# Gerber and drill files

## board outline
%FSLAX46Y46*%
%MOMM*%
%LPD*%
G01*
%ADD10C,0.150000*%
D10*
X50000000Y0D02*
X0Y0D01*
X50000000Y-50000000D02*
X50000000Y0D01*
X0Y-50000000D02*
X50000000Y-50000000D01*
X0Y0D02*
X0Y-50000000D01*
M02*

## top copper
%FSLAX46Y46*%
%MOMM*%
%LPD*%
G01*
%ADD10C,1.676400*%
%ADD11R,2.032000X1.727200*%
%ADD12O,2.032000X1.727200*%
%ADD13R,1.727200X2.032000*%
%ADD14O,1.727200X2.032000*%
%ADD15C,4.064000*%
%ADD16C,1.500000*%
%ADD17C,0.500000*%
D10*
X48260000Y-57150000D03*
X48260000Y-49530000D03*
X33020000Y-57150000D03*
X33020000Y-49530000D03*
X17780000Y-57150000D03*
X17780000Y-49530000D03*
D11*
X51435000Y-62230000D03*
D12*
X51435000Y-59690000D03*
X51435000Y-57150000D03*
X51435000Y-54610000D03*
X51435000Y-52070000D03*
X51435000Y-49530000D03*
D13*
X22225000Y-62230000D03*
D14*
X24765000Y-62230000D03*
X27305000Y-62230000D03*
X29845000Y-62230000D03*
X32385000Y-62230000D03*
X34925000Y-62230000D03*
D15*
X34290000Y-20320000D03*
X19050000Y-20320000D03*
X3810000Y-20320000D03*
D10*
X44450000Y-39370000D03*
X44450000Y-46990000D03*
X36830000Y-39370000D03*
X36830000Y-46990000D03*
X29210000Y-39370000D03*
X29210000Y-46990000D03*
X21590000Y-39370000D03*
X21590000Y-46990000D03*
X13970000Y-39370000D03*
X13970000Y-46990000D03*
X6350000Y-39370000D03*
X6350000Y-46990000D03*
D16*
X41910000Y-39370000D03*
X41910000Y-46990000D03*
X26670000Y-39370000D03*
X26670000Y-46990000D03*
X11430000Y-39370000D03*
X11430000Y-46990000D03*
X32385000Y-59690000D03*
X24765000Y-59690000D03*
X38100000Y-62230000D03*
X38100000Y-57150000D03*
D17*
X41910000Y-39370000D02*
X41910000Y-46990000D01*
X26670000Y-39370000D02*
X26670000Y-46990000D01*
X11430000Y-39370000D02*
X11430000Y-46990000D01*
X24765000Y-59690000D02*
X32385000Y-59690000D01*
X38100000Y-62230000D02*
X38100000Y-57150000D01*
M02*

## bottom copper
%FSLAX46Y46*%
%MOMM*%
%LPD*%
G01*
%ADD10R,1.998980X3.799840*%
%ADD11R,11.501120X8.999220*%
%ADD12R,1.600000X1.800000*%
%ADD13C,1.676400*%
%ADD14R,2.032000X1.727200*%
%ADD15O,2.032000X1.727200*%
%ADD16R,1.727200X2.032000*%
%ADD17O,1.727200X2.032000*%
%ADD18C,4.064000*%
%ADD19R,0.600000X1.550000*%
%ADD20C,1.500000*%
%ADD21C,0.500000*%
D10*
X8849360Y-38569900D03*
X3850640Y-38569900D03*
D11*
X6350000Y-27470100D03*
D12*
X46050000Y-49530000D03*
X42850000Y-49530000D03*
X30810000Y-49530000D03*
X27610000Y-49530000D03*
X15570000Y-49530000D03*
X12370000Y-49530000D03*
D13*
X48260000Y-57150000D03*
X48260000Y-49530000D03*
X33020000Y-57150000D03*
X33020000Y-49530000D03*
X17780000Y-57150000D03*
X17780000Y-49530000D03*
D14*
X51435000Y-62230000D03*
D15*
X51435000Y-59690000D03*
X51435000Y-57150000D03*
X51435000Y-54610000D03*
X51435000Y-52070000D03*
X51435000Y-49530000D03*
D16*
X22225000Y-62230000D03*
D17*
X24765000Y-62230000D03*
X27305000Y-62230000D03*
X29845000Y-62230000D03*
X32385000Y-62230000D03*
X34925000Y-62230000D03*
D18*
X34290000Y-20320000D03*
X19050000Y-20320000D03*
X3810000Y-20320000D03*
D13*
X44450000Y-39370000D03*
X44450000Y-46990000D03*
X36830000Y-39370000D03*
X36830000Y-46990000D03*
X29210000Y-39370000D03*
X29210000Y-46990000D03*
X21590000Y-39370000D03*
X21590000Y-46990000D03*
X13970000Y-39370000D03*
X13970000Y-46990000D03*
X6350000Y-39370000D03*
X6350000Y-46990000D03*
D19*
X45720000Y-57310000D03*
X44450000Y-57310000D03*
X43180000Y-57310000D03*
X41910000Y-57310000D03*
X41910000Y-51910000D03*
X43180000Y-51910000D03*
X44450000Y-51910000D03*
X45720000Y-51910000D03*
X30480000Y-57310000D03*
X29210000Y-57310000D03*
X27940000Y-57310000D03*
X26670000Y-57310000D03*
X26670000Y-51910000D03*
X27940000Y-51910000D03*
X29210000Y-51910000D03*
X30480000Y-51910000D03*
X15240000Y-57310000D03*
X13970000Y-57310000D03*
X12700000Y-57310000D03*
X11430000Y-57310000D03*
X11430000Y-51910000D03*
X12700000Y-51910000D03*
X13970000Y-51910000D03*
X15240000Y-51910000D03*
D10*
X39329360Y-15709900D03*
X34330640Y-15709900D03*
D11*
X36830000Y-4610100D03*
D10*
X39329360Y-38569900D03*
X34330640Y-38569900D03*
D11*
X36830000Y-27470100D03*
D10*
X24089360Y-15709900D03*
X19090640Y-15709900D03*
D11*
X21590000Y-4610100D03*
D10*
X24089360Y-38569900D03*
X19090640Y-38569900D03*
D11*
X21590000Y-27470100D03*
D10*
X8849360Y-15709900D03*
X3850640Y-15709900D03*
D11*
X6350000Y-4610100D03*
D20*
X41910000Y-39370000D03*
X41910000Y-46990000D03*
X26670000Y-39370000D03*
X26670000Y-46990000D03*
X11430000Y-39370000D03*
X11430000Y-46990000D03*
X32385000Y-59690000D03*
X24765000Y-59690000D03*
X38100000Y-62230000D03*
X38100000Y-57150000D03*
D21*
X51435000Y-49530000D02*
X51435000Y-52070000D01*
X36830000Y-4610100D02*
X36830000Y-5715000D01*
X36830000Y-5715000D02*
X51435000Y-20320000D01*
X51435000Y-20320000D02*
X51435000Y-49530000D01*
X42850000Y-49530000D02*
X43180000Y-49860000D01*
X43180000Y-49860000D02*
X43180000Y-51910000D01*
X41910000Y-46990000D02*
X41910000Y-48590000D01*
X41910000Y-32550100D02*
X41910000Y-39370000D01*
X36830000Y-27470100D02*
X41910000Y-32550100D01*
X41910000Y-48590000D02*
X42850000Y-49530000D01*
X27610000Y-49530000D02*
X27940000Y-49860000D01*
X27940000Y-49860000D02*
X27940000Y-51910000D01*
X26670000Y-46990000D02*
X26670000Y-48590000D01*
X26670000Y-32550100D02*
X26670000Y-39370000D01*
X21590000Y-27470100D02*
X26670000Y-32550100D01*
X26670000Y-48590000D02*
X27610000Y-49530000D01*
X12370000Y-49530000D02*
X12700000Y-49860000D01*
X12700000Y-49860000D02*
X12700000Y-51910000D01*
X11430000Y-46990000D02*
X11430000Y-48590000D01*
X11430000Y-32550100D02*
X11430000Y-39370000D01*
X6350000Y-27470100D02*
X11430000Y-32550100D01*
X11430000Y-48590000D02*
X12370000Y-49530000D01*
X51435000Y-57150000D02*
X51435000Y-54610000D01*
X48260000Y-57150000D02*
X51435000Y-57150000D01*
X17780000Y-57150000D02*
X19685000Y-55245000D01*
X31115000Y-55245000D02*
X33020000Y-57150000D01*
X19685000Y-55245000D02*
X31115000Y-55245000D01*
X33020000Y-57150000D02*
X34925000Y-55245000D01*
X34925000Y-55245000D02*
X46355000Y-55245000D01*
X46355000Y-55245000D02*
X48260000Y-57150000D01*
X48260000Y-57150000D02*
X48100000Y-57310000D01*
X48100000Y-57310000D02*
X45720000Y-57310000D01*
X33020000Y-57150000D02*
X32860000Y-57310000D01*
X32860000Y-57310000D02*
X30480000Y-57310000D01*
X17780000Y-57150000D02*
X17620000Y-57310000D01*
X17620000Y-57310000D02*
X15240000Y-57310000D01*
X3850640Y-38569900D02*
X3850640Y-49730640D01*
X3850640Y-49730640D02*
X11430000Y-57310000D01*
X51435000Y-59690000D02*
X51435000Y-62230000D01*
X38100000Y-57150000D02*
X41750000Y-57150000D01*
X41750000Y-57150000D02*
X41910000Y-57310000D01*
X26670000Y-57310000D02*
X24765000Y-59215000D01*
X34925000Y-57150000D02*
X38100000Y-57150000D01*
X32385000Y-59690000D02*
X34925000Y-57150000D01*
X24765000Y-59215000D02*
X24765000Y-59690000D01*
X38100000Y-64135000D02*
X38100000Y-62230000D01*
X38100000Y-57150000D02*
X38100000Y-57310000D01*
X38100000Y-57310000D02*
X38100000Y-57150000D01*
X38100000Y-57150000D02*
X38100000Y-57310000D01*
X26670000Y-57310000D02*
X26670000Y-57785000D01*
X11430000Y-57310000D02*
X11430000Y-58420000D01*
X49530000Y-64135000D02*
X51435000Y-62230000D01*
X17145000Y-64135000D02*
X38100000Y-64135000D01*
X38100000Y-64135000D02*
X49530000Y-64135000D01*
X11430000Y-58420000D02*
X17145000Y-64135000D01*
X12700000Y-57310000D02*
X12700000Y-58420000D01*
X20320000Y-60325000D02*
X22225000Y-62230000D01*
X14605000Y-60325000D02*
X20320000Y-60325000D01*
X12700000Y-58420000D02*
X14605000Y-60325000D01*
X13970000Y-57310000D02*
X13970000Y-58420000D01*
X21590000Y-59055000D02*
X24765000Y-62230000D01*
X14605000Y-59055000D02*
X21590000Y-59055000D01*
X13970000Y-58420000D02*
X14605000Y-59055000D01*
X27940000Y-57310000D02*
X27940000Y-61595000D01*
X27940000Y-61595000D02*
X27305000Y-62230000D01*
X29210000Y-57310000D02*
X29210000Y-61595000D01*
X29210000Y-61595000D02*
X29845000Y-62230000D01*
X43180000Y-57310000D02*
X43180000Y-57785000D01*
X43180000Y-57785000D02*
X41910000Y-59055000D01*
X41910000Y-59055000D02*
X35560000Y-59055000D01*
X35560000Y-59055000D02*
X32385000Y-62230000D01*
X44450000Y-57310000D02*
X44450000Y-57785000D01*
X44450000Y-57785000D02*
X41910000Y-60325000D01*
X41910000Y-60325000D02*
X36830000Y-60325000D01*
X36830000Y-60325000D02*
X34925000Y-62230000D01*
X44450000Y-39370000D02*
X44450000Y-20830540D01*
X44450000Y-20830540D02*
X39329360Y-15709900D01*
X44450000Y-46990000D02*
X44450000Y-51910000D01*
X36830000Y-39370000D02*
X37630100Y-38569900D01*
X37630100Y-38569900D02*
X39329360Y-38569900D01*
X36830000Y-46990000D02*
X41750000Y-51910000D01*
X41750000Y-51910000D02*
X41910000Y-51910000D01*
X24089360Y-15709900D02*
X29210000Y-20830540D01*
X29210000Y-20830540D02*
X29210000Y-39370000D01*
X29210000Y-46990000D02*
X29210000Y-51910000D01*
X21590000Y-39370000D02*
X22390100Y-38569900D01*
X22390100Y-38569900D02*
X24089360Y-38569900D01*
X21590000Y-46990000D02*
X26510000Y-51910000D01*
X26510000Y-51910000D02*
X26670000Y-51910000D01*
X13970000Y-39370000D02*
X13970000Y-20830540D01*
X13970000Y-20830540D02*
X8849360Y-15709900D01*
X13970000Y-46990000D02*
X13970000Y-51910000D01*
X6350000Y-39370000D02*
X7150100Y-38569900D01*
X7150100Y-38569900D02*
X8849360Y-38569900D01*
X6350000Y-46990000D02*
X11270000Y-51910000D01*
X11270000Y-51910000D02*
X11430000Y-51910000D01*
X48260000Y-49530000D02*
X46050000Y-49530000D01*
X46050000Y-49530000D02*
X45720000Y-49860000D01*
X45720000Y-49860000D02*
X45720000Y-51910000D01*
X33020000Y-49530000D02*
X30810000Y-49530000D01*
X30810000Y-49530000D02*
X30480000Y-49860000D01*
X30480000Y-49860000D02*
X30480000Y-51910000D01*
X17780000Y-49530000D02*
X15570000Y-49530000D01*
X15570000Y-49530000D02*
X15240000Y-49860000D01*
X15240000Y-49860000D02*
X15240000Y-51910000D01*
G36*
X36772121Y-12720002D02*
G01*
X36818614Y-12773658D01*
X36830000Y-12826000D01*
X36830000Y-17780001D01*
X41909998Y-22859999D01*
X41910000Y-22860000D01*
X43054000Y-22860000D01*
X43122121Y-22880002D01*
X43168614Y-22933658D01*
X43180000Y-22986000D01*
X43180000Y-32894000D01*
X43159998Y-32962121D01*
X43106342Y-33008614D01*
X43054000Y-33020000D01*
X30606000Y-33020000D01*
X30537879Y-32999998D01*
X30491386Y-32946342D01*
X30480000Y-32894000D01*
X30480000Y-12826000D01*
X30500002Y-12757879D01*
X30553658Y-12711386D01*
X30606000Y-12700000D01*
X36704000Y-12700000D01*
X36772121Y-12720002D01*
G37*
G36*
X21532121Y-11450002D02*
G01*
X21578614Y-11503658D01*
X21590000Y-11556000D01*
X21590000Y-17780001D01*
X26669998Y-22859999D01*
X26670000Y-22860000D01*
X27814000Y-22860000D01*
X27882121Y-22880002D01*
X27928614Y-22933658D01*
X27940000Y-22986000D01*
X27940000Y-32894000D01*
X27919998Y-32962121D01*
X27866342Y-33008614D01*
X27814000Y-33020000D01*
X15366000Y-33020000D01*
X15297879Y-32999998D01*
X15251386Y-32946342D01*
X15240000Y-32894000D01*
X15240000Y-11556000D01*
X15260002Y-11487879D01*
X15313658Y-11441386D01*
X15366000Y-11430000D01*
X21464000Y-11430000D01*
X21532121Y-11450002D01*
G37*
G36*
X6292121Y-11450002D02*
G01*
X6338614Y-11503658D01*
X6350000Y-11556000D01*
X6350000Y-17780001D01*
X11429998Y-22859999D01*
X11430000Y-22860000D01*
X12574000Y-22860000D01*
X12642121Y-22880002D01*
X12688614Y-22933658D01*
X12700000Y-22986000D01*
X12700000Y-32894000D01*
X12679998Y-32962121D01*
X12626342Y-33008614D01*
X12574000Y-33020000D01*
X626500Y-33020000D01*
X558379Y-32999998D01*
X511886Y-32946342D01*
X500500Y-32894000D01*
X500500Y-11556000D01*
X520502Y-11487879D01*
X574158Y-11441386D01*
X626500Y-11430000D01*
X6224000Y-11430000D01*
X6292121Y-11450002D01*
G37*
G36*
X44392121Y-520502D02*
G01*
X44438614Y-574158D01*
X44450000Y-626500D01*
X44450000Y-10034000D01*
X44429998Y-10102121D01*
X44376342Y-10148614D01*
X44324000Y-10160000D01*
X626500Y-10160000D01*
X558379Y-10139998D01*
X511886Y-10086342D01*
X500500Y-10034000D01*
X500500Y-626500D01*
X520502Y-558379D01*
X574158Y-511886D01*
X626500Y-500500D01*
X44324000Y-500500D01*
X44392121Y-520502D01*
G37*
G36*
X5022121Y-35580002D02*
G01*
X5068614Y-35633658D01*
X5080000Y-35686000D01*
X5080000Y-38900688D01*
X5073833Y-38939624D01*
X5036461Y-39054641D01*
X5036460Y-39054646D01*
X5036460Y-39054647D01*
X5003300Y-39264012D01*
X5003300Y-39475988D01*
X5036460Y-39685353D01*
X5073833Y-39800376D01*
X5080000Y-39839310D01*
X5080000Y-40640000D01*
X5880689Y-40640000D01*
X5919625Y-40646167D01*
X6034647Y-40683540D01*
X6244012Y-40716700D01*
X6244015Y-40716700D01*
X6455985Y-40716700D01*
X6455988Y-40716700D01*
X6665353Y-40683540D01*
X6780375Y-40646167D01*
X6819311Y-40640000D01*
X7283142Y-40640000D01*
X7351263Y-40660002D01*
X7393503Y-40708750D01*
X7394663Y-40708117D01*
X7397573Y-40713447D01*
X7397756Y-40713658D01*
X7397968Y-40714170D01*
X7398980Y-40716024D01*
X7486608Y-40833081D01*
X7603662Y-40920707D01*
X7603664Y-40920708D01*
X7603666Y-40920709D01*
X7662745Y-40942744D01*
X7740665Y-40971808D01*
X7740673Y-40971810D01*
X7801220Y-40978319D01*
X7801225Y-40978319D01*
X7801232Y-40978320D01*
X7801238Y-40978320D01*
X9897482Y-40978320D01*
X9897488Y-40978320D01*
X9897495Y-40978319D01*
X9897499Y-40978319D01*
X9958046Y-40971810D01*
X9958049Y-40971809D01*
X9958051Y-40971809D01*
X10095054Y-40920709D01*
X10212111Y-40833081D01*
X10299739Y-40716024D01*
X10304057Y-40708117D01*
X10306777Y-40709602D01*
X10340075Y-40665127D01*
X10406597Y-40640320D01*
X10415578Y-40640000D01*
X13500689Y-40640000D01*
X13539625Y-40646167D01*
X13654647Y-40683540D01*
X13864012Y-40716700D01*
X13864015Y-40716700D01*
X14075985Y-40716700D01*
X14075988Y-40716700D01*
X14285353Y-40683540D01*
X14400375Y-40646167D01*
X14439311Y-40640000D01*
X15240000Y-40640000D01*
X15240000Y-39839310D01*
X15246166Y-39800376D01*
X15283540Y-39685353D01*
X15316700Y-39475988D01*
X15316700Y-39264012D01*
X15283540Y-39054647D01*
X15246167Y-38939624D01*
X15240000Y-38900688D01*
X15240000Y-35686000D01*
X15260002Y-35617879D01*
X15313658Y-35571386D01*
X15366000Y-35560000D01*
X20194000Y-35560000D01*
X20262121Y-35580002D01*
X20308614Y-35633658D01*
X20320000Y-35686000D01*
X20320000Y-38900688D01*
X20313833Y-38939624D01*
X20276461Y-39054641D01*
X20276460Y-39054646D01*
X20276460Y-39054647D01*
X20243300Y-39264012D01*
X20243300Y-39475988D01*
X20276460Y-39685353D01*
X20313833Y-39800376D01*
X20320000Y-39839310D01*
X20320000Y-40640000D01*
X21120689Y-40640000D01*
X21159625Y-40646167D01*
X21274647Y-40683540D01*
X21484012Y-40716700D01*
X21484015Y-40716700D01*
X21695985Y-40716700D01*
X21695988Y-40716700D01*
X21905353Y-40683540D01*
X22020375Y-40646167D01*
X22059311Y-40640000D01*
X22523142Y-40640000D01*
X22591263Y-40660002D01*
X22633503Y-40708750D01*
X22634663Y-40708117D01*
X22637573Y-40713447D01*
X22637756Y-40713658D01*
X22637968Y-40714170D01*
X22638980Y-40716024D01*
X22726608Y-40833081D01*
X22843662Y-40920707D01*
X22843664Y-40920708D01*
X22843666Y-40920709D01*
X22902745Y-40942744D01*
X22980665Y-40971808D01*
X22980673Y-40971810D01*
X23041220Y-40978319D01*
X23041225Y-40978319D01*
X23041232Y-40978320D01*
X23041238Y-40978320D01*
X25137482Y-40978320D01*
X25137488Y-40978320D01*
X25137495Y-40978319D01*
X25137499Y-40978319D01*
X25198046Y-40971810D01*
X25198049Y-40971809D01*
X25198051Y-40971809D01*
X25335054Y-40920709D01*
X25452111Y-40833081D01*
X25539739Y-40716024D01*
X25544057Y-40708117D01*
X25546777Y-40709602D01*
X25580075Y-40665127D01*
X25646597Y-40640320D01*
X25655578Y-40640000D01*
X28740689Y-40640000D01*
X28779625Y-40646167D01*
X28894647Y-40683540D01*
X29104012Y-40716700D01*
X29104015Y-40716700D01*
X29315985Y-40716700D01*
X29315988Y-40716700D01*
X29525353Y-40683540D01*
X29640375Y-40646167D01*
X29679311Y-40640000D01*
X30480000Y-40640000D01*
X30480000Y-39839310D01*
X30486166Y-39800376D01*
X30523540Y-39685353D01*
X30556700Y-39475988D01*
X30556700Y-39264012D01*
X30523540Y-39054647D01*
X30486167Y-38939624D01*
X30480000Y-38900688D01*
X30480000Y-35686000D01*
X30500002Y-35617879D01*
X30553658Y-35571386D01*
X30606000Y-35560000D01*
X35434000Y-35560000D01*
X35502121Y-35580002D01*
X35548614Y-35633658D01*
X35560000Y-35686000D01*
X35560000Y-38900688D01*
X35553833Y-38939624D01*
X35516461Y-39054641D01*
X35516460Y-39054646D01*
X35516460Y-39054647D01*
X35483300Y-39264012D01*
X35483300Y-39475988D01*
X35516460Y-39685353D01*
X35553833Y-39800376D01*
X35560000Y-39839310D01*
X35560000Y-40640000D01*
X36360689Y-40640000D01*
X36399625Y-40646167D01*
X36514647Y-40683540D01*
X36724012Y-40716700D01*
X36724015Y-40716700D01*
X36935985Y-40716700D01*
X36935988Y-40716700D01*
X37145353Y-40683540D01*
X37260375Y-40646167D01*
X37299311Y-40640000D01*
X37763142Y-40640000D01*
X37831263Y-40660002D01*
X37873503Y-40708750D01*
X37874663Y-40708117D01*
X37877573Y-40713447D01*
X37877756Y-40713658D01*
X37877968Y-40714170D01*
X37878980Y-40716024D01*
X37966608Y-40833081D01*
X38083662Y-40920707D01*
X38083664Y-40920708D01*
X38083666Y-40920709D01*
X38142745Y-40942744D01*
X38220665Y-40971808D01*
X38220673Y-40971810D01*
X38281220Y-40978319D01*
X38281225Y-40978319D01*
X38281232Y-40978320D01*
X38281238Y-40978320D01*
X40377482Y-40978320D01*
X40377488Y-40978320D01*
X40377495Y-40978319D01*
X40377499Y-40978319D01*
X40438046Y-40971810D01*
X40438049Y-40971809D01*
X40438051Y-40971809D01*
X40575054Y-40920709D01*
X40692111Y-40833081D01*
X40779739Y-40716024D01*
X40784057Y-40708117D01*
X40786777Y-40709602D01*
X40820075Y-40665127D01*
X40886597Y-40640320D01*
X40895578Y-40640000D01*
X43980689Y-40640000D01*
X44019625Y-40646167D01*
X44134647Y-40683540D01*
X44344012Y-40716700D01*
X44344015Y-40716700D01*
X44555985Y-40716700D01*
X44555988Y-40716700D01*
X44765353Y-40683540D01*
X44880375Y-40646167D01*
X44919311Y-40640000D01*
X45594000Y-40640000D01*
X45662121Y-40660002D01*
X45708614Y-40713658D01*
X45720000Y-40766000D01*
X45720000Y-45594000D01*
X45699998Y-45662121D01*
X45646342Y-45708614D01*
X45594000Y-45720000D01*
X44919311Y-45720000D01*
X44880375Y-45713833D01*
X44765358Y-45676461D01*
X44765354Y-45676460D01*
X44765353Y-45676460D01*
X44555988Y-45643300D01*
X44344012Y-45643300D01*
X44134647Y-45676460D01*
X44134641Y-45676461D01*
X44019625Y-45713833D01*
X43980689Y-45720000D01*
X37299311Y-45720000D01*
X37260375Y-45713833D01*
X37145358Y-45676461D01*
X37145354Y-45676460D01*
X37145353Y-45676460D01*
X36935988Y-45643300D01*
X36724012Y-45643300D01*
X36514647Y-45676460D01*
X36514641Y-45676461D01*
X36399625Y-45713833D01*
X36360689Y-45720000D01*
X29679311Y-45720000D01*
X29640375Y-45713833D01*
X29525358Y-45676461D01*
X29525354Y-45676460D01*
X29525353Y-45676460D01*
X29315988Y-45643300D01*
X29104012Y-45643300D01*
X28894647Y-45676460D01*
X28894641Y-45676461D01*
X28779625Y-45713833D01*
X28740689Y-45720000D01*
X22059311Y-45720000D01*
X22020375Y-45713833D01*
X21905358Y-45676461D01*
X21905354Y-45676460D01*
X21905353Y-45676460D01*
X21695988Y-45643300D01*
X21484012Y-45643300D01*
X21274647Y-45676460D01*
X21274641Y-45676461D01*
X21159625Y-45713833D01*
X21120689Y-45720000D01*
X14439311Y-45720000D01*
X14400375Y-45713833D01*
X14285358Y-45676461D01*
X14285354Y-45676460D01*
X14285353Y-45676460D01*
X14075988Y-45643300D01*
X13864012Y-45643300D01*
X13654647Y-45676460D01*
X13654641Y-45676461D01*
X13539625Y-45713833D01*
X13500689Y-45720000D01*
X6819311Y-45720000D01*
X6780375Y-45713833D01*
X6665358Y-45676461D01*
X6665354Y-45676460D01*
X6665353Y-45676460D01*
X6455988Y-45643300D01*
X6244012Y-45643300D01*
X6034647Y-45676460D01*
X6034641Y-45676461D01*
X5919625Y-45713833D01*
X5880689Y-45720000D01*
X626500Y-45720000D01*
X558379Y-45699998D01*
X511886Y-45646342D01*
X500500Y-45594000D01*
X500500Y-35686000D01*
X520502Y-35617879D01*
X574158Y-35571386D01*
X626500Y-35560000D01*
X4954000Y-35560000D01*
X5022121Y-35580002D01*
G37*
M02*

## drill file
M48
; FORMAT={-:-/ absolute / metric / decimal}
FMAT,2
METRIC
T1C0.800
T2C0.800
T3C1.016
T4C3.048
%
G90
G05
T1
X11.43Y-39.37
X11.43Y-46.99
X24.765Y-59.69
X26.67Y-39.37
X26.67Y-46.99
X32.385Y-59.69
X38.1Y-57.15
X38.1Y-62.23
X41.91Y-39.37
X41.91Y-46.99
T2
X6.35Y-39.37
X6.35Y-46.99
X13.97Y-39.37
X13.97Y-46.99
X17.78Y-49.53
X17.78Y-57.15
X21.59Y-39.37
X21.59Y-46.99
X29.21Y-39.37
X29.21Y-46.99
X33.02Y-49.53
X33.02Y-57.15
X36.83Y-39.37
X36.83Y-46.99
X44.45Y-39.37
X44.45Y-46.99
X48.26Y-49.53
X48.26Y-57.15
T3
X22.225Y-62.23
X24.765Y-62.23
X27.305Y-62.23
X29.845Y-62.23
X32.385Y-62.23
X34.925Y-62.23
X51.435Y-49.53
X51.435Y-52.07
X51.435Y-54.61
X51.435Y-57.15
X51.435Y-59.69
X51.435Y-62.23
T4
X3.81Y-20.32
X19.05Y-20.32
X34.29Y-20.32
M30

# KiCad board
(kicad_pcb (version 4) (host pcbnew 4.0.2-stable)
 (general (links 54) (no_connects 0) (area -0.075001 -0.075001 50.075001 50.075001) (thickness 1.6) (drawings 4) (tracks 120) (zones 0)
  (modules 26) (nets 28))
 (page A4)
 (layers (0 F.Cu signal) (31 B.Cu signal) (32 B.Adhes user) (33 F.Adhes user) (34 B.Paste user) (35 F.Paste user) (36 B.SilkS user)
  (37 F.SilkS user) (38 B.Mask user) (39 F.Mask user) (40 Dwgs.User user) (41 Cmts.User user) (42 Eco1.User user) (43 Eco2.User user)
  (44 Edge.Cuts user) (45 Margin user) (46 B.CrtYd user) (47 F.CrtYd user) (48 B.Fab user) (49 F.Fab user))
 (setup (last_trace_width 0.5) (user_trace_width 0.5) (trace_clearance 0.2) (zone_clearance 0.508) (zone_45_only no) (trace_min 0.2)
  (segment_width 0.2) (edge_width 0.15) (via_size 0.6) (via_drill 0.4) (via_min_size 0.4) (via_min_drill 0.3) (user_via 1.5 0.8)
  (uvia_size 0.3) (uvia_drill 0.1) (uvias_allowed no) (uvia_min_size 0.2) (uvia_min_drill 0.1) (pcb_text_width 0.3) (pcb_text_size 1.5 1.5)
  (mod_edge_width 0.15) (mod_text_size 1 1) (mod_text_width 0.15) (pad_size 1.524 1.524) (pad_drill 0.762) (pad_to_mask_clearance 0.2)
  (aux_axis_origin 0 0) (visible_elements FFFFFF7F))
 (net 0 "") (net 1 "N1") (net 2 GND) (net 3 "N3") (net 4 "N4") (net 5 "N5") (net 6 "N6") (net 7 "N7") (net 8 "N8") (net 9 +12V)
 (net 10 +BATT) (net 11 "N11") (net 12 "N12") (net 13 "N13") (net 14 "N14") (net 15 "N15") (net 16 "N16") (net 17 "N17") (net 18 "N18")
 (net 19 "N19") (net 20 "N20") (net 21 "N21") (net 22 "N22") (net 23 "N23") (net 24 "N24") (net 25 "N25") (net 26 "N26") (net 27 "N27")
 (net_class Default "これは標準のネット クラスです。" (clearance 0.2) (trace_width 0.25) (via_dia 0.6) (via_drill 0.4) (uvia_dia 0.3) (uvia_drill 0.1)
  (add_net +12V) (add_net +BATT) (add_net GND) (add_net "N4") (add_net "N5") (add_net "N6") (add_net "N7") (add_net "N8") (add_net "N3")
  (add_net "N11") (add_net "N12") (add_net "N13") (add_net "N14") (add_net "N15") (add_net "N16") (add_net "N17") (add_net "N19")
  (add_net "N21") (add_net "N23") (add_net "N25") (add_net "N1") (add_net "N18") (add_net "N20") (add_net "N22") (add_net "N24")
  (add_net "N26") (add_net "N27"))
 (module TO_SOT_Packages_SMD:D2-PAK (layer B.Cu) (at 6.35 33.02 180)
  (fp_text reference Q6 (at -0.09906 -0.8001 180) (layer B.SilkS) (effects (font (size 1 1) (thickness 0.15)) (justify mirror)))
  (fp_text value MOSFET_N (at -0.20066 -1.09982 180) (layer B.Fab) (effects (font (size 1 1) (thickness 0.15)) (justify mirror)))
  (pad G smd rect (at -2.49936 -5.5499 180) (size 1.99898 3.79984) (layers B.Cu B.Paste B.Mask) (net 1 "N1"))
  (pad S smd rect (at 2.49936 -5.5499 180) (size 1.99898 3.79984) (layers B.Cu B.Paste B.Mask) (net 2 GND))
  (pad D smd rect (at 0 5.5499 180) (size 11.50112 8.99922) (layers B.Cu B.Paste B.Mask) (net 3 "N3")))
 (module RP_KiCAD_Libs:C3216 (layer B.Cu) (at 44.45 49.53 180)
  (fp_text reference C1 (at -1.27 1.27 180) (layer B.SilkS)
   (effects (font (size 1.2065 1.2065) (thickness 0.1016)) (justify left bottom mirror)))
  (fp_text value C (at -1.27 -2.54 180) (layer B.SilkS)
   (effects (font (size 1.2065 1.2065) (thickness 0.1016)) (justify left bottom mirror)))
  (pad 1 smd rect (at -1.6 0 180) (size 1.6 1.8) (layers B.Cu B.Paste B.Mask) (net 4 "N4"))
  (pad 2 smd rect (at 1.6 0 180) (size 1.6 1.8) (layers B.Cu B.Paste B.Mask) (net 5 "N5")))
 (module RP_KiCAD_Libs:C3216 (layer B.Cu) (at 29.21 49.53 180)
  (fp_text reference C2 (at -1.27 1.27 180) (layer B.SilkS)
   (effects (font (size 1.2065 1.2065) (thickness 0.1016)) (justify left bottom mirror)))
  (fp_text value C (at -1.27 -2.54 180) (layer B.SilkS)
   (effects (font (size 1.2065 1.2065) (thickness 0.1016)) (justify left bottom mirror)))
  (pad 1 smd rect (at -1.6 0 180) (size 1.6 1.8) (layers B.Cu B.Paste B.Mask) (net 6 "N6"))
  (pad 2 smd rect (at 1.6 0 180) (size 1.6 1.8) (layers B.Cu B.Paste B.Mask) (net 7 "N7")))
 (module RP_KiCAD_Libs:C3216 (layer B.Cu) (at 13.97 49.53 180)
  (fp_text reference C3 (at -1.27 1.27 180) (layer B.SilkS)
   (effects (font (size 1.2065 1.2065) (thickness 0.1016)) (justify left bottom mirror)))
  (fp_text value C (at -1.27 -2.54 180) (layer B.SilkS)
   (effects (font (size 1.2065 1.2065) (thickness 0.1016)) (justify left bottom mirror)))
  (pad 1 smd rect (at -1.6 0 180) (size 1.6 1.8) (layers B.Cu B.Paste B.Mask) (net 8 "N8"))
  (pad 2 smd rect (at 1.6 0 180) (size 1.6 1.8) (layers B.Cu B.Paste B.Mask) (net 3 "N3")))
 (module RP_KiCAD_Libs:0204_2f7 (layer F.Cu) (at 48.26 53.34 90)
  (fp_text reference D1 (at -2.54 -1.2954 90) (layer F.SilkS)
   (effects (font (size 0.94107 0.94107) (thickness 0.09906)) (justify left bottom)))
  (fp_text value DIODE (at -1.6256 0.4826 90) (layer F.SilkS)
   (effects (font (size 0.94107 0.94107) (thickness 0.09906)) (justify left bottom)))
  (pad 1 thru_hole circle (at -3.81 0 90) (size 1.6764 1.6764) (drill 0.8) (layers *.Cu *.Mask) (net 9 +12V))
  (pad 2 thru_hole circle (at 3.81 0 90) (size 1.6764 1.6764) (drill 0.8) (layers *.Cu *.Mask) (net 4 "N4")))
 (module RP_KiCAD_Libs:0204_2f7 (layer F.Cu) (at 33.02 53.34 90)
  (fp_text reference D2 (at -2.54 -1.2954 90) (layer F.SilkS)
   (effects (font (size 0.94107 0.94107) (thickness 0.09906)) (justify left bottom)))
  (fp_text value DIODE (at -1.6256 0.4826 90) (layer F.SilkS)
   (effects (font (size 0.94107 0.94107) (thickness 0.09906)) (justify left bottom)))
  (pad 1 thru_hole circle (at -3.81 0 90) (size 1.6764 1.6764) (drill 0.8) (layers *.Cu *.Mask) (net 9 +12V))
  (pad 2 thru_hole circle (at 3.81 0 90) (size 1.6764 1.6764) (drill 0.8) (layers *.Cu *.Mask) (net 6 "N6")))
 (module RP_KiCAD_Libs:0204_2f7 (layer F.Cu) (at 17.78 53.34 90)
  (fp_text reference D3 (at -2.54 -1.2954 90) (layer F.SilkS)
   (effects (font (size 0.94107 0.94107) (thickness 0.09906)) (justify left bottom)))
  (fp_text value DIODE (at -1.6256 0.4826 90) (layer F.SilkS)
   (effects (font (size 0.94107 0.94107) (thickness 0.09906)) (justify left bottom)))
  (pad 1 thru_hole circle (at -3.81 0 90) (size 1.6764 1.6764) (drill 0.8) (layers *.Cu *.Mask) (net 9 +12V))
  (pad 2 thru_hole circle (at 3.81 0 90) (size 1.6764 1.6764) (drill 0.8) (layers *.Cu *.Mask) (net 8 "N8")))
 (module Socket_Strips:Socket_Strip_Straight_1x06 (layer F.Cu) (at 51.435 62.23 90)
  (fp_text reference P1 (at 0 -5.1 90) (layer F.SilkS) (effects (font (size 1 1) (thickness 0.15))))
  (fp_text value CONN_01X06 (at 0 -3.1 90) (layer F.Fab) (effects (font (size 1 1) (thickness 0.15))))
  (pad 1 thru_hole rect (at 0 0 90) (size 1.7272 2.032) (drill 1.016) (layers *.Cu *.Mask F.SilkS) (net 2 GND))
  (pad 2 thru_hole oval (at 2.54 0 90) (size 1.7272 2.032) (drill 1.016) (layers *.Cu *.Mask F.SilkS) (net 2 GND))
  (pad 3 thru_hole oval (at 5.08 0 90) (size 1.7272 2.032) (drill 1.016) (layers *.Cu *.Mask F.SilkS) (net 9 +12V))
  (pad 4 thru_hole oval (at 7.62 0 90) (size 1.7272 2.032) (drill 1.016) (layers *.Cu *.Mask F.SilkS) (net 9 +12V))
  (pad 5 thru_hole oval (at 10.16 0 90) (size 1.7272 2.032) (drill 1.016) (layers *.Cu *.Mask F.SilkS) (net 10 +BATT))
  (pad 6 thru_hole oval (at 12.7 0 90) (size 1.7272 2.032) (drill 1.016) (layers *.Cu *.Mask F.SilkS) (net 10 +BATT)))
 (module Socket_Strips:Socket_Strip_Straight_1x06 (layer F.Cu) (at 22.225 62.23)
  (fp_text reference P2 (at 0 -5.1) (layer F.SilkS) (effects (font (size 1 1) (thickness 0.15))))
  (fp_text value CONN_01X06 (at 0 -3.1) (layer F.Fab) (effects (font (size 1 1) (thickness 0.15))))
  (pad 1 thru_hole rect (at 0 0) (size 1.7272 2.032) (drill 1.016) (layers *.Cu *.Mask F.SilkS) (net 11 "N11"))
  (pad 2 thru_hole oval (at 2.54 0) (size 1.7272 2.032) (drill 1.016) (layers *.Cu *.Mask F.SilkS) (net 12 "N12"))
  (pad 3 thru_hole oval (at 5.08 0) (size 1.7272 2.032) (drill 1.016) (layers *.Cu *.Mask F.SilkS) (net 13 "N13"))
  (pad 4 thru_hole oval (at 7.62 0) (size 1.7272 2.032) (drill 1.016) (layers *.Cu *.Mask F.SilkS) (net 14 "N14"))
  (pad 5 thru_hole oval (at 10.16 0) (size 1.7272 2.032) (drill 1.016) (layers *.Cu *.Mask F.SilkS) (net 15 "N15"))
  (pad 6 thru_hole oval (at 12.7 0) (size 1.7272 2.032) (drill 1.016) (layers *.Cu *.Mask F.SilkS) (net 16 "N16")))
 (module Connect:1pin (layer F.Cu) (at 34.29 20.32)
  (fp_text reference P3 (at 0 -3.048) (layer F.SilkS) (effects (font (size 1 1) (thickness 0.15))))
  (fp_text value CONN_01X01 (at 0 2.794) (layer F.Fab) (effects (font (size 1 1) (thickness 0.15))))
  (pad 1 thru_hole circle (at 0 0) (size 4.064 4.064) (drill 3.048) (layers *.Cu *.Mask F.SilkS) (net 5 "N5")))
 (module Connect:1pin (layer F.Cu) (at 19.05 20.32)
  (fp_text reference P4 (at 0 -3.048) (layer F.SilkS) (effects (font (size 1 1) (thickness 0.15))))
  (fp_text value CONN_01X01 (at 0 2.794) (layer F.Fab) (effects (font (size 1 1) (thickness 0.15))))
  (pad 1 thru_hole circle (at 0 0) (size 4.064 4.064) (drill 3.048) (layers *.Cu *.Mask F.SilkS) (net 7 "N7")))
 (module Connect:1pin (layer F.Cu) (at 3.81 20.32)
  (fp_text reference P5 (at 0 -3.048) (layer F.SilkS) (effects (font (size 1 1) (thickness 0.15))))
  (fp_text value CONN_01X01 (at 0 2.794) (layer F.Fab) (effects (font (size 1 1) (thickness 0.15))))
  (pad 1 thru_hole circle (at 0 0) (size 4.064 4.064) (drill 3.048) (layers *.Cu *.Mask F.SilkS) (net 3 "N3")))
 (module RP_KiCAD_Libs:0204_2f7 (layer F.Cu) (at 44.45 43.18 270)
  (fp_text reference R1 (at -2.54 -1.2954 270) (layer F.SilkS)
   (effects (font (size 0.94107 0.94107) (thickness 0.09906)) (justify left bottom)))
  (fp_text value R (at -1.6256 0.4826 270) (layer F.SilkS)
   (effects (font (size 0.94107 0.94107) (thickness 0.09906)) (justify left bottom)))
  (pad 1 thru_hole circle (at -3.81 0 270) (size 1.6764 1.6764) (drill 0.8) (layers *.Cu *.Mask) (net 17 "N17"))
  (pad 2 thru_hole circle (at 3.81 0 270) (size 1.6764 1.6764) (drill 0.8) (layers *.Cu *.Mask) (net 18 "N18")))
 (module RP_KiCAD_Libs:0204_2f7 (layer F.Cu) (at 36.83 43.18 270)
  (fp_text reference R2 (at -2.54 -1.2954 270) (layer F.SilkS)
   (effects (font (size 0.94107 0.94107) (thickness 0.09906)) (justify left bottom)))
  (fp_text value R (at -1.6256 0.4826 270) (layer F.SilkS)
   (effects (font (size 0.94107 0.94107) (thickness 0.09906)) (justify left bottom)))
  (pad 1 thru_hole circle (at -3.81 0 270) (size 1.6764 1.6764) (drill 0.8) (layers *.Cu *.Mask) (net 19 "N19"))
  (pad 2 thru_hole circle (at 3.81 0 270) (size 1.6764 1.6764) (drill 0.8) (layers *.Cu *.Mask) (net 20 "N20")))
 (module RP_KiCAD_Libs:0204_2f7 (layer F.Cu) (at 29.21 43.18 270)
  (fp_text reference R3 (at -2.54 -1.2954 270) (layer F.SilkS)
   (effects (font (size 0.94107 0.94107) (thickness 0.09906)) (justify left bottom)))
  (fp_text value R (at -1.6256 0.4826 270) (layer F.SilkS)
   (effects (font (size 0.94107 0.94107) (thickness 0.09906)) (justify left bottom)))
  (pad 1 thru_hole circle (at -3.81 0 270) (size 1.6764 1.6764) (drill 0.8) (layers *.Cu *.Mask) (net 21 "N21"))
  (pad 2 thru_hole circle (at 3.81 0 270) (size 1.6764 1.6764) (drill 0.8) (layers *.Cu *.Mask) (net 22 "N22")))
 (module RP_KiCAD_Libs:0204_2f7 (layer F.Cu) (at 21.59 43.18 270)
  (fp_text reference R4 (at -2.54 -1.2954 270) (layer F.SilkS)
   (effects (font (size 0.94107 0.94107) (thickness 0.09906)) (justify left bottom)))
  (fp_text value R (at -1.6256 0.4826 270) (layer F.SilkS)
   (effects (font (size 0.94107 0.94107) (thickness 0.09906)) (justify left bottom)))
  (pad 1 thru_hole circle (at -3.81 0 270) (size 1.6764 1.6764) (drill 0.8) (layers *.Cu *.Mask) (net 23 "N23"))
  (pad 2 thru_hole circle (at 3.81 0 270) (size 1.6764 1.6764) (drill 0.8) (layers *.Cu *.Mask) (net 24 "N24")))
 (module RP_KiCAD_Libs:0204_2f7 (layer F.Cu) (at 13.97 43.18 270)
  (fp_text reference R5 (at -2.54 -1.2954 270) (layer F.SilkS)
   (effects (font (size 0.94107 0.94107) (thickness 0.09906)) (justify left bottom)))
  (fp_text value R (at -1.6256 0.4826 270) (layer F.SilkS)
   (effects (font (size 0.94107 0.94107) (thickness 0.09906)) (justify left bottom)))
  (pad 1 thru_hole circle (at -3.81 0 270) (size 1.6764 1.6764) (drill 0.8) (layers *.Cu *.Mask) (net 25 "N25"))
  (pad 2 thru_hole circle (at 3.81 0 270) (size 1.6764 1.6764) (drill 0.8) (layers *.Cu *.Mask) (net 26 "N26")))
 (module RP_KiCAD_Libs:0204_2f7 (layer F.Cu) (at 6.35 43.18 270)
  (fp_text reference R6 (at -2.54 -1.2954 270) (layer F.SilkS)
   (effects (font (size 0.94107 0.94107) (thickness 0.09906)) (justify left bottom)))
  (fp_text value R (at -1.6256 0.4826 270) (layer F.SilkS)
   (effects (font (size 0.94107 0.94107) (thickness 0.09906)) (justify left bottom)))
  (pad 1 thru_hole circle (at -3.81 0 270) (size 1.6764 1.6764) (drill 0.8) (layers *.Cu *.Mask) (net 1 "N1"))
  (pad 2 thru_hole circle (at 3.81 0 270) (size 1.6764 1.6764) (drill 0.8) (layers *.Cu *.Mask) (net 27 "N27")))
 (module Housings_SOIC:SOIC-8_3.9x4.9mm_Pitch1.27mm (layer B.Cu) (at 43.815 54.61 90)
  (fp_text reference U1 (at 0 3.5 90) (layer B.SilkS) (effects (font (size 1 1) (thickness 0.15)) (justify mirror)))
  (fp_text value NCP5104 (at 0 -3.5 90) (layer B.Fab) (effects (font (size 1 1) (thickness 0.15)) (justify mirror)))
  (pad 1 smd rect (at -2.7 1.905 90) (size 1.55 0.6) (layers B.Cu B.Paste B.Mask) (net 9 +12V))
  (pad 2 smd rect (at -2.7 0.635 90) (size 1.55 0.6) (layers B.Cu B.Paste B.Mask) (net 16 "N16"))
  (pad 3 smd rect (at -2.7 -0.635 90) (size 1.55 0.6) (layers B.Cu B.Paste B.Mask) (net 15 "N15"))
  (pad 4 smd rect (at -2.7 -1.905 90) (size 1.55 0.6) (layers B.Cu B.Paste B.Mask) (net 2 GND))
  (pad 5 smd rect (at 2.7 -1.905 90) (size 1.55 0.6) (layers B.Cu B.Paste B.Mask) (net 20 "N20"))
  (pad 6 smd rect (at 2.7 -0.635 90) (size 1.55 0.6) (layers B.Cu B.Paste B.Mask) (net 5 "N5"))
  (pad 7 smd rect (at 2.7 0.635 90) (size 1.55 0.6) (layers B.Cu B.Paste B.Mask) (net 18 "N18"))
  (pad 8 smd rect (at 2.7 1.905 90) (size 1.55 0.6) (layers B.Cu B.Paste B.Mask) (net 4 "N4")))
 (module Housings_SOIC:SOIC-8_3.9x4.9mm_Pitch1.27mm (layer B.Cu) (at 28.575 54.61 90)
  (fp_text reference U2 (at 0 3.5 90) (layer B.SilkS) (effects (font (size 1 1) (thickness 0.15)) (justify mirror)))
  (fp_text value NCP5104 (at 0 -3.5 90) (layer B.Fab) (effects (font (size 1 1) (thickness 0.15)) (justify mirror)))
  (pad 1 smd rect (at -2.7 1.905 90) (size 1.55 0.6) (layers B.Cu B.Paste B.Mask) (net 9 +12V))
  (pad 2 smd rect (at -2.7 0.635 90) (size 1.55 0.6) (layers B.Cu B.Paste B.Mask) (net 14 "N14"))
  (pad 3 smd rect (at -2.7 -0.635 90) (size 1.55 0.6) (layers B.Cu B.Paste B.Mask) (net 13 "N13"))
  (pad 4 smd rect (at -2.7 -1.905 90) (size 1.55 0.6) (layers B.Cu B.Paste B.Mask) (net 2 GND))
  (pad 5 smd rect (at 2.7 -1.905 90) (size 1.55 0.6) (layers B.Cu B.Paste B.Mask) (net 24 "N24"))
  (pad 6 smd rect (at 2.7 -0.635 90) (size 1.55 0.6) (layers B.Cu B.Paste B.Mask) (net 7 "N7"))
  (pad 7 smd rect (at 2.7 0.635 90) (size 1.55 0.6) (layers B.Cu B.Paste B.Mask) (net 22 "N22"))
  (pad 8 smd rect (at 2.7 1.905 90) (size 1.55 0.6) (layers B.Cu B.Paste B.Mask) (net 6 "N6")))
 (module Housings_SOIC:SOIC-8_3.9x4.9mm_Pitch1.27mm (layer B.Cu) (at 13.335 54.61 90)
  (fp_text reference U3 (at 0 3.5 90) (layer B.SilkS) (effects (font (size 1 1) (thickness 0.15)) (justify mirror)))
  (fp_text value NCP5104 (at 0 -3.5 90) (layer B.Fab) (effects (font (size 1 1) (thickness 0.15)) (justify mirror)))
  (pad 1 smd rect (at -2.7 1.905 90) (size 1.55 0.6) (layers B.Cu B.Paste B.Mask) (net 9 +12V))
  (pad 2 smd rect (at -2.7 0.635 90) (size 1.55 0.6) (layers B.Cu B.Paste B.Mask) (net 12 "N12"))
  (pad 3 smd rect (at -2.7 -0.635 90) (size 1.55 0.6) (layers B.Cu B.Paste B.Mask) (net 11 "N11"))
  (pad 4 smd rect (at -2.7 -1.905 90) (size 1.55 0.6) (layers B.Cu B.Paste B.Mask) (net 2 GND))
  (pad 5 smd rect (at 2.7 -1.905 90) (size 1.55 0.6) (layers B.Cu B.Paste B.Mask) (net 27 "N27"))
  (pad 6 smd rect (at 2.7 -0.635 90) (size 1.55 0.6) (layers B.Cu B.Paste B.Mask) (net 3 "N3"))
  (pad 7 smd rect (at 2.7 0.635 90) (size 1.55 0.6) (layers B.Cu B.Paste B.Mask) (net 26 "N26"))
  (pad 8 smd rect (at 2.7 1.905 90) (size 1.55 0.6) (layers B.Cu B.Paste B.Mask) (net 8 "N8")))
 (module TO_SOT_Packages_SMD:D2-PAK (layer B.Cu) (at 36.83 10.16 180)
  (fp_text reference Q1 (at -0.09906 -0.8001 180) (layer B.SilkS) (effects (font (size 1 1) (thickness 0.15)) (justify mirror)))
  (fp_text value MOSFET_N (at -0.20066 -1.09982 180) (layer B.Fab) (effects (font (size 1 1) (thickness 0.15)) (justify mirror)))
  (pad G smd rect (at -2.49936 -5.5499 180) (size 1.99898 3.79984) (layers B.Cu B.Paste B.Mask) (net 17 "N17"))
  (pad S smd rect (at 2.49936 -5.5499 180) (size 1.99898 3.79984) (layers B.Cu B.Paste B.Mask) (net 5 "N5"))
  (pad D smd rect (at 0 5.5499 180) (size 11.50112 8.99922) (layers B.Cu B.Paste B.Mask) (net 10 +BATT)))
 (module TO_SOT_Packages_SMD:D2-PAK (layer B.Cu) (at 36.83 33.02 180)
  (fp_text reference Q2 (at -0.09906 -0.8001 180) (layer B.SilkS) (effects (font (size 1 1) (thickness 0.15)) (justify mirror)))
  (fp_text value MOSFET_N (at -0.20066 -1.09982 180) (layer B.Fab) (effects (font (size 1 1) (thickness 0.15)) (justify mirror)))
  (pad G smd rect (at -2.49936 -5.5499 180) (size 1.99898 3.79984) (layers B.Cu B.Paste B.Mask) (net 19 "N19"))
  (pad S smd rect (at 2.49936 -5.5499 180) (size 1.99898 3.79984) (layers B.Cu B.Paste B.Mask) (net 2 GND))
  (pad D smd rect (at 0 5.5499 180) (size 11.50112 8.99922) (layers B.Cu B.Paste B.Mask) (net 5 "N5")))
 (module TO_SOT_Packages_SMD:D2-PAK (layer B.Cu) (at 21.59 10.16 180)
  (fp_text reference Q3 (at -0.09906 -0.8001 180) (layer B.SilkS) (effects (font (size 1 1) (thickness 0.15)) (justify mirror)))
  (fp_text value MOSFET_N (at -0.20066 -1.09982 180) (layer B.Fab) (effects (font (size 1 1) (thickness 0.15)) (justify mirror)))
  (pad G smd rect (at -2.49936 -5.5499 180) (size 1.99898 3.79984) (layers B.Cu B.Paste B.Mask) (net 21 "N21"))
  (pad S smd rect (at 2.49936 -5.5499 180) (size 1.99898 3.79984) (layers B.Cu B.Paste B.Mask) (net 7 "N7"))
  (pad D smd rect (at 0 5.5499 180) (size 11.50112 8.99922) (layers B.Cu B.Paste B.Mask) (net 10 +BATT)))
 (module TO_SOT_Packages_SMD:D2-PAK (layer B.Cu) (at 21.59 33.02 180)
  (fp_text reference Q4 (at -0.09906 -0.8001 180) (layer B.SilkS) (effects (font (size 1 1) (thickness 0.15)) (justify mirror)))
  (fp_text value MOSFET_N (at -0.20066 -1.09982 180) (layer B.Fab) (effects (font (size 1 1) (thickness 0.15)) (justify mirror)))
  (pad G smd rect (at -2.49936 -5.5499 180) (size 1.99898 3.79984) (layers B.Cu B.Paste B.Mask) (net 23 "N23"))
  (pad S smd rect (at 2.49936 -5.5499 180) (size 1.99898 3.79984) (layers B.Cu B.Paste B.Mask) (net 2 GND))
  (pad D smd rect (at 0 5.5499 180) (size 11.50112 8.99922) (layers B.Cu B.Paste B.Mask) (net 7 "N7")))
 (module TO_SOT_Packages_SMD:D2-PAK (layer B.Cu) (at 6.35 10.16 180)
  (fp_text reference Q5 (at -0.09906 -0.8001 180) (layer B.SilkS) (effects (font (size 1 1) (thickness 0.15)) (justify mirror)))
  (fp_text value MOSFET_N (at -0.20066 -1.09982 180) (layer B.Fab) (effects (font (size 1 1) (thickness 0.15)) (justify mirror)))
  (pad G smd rect (at -2.49936 -5.5499 180) (size 1.99898 3.79984) (layers B.Cu B.Paste B.Mask) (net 25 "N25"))
  (pad S smd rect (at 2.49936 -5.5499 180) (size 1.99898 3.79984) (layers B.Cu B.Paste B.Mask) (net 3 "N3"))
  (pad D smd rect (at 0 5.5499 180) (size 11.50112 8.99922) (layers B.Cu B.Paste B.Mask) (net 10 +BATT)))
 (gr_line (start 50 0) (end 0 0) (angle 90) (layer Edge.Cuts) (width 0.15))
 (gr_line (start 50 50) (end 50 0) (angle 90) (layer Edge.Cuts) (width 0.15))
 (gr_line (start 0 50) (end 50 50) (angle 90) (layer Edge.Cuts) (width 0.15))
 (gr_line (start 0 0) (end 0 50) (angle 90) (layer Edge.Cuts) (width 0.15))
 (segment (start 51.435 49.53) (end 51.435 52.07) (width 0.5) (layer B.Cu) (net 10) (status C00000))
 (segment (start 36.83 4.6101) (end 36.83 5.715) (width 0.5) (layer B.Cu) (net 10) (status C00000))
 (segment (start 36.83 5.715) (end 51.435 20.32) (width 0.5) (layer B.Cu) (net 10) (status 400000))
 (segment (start 51.435 20.32) (end 51.435 49.53) (width 0.5) (layer B.Cu) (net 10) (status 800000))
 (segment (start 42.85 49.53) (end 43.18 49.86) (width 0.5) (layer B.Cu) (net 5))
 (segment (start 43.18 49.86) (end 43.18 51.91) (width 0.5) (layer B.Cu) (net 5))
 (segment (start 41.91 46.99) (end 41.91 48.59) (width 0.5) (layer B.Cu) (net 5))
 (segment (start 41.91 32.5501) (end 41.91 39.37) (width 0.5) (layer B.Cu) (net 5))
 (via (at 41.91 39.37) (size 1.5) (drill 0.8) (layers F.Cu B.Cu) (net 5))
 (segment (start 41.91 39.37) (end 41.91 46.99) (width 0.5) (layer F.Cu) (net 5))
 (via (at 41.91 46.99) (size 1.5) (drill 0.8) (layers F.Cu B.Cu) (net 5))
 (segment (start 36.83 27.4701) (end 41.91 32.5501) (width 0.5) (layer B.Cu) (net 5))
 (segment (start 41.91 48.59) (end 42.85 49.53) (width 0.5) (layer B.Cu) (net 5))
 (segment (start 27.61 49.53) (end 27.94 49.86) (width 0.5) (layer B.Cu) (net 7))
 (segment (start 27.94 49.86) (end 27.94 51.91) (width 0.5) (layer B.Cu) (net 7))
 (segment (start 26.67 46.99) (end 26.67 48.59) (width 0.5) (layer B.Cu) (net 7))
 (segment (start 26.67 32.5501) (end 26.67 39.37) (width 0.5) (layer B.Cu) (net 7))
 (via (at 26.67 39.37) (size 1.5) (drill 0.8) (layers F.Cu B.Cu) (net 7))
 (segment (start 26.67 39.37) (end 26.67 46.99) (width 0.5) (layer F.Cu) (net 7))
 (via (at 26.67 46.99) (size 1.5) (drill 0.8) (layers F.Cu B.Cu) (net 7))
 (segment (start 21.59 27.4701) (end 26.67 32.5501) (width 0.5) (layer B.Cu) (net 7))
 (segment (start 26.67 48.59) (end 27.61 49.53) (width 0.5) (layer B.Cu) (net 7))
 (segment (start 12.37 49.53) (end 12.7 49.86) (width 0.5) (layer B.Cu) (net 3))
 (segment (start 12.7 49.86) (end 12.7 51.91) (width 0.5) (layer B.Cu) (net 3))
 (segment (start 11.43 46.99) (end 11.43 48.59) (width 0.5) (layer B.Cu) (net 3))
 (segment (start 11.43 32.5501) (end 11.43 39.37) (width 0.5) (layer B.Cu) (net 3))
 (via (at 11.43 39.37) (size 1.5) (drill 0.8) (layers F.Cu B.Cu) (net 3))
 (segment (start 11.43 39.37) (end 11.43 46.99) (width 0.5) (layer F.Cu) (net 3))
 (via (at 11.43 46.99) (size 1.5) (drill 0.8) (layers F.Cu B.Cu) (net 3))
 (segment (start 6.35 27.4701) (end 11.43 32.5501) (width 0.5) (layer B.Cu) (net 3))
 (segment (start 11.43 48.59) (end 12.37 49.53) (width 0.5) (layer B.Cu) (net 3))
 (segment (start 51.435 57.15) (end 51.435 54.61) (width 0.5) (layer B.Cu) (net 9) (status C00000))
 (segment (start 48.26 57.15) (end 51.435 57.15) (width 0.5) (layer B.Cu) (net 9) (status C00000))
 (segment (start 17.78 57.15) (end 19.685 55.245) (width 0.5) (layer B.Cu) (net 9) (status 400000))
 (segment (start 31.115 55.245) (end 33.02 57.15) (width 0.5) (layer B.Cu) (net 9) (status 800000))
 (segment (start 19.685 55.245) (end 31.115 55.245) (width 0.5) (layer B.Cu) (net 9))
 (segment (start 33.02 57.15) (end 34.925 55.245) (width 0.5) (layer B.Cu) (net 9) (status 400000))
 (segment (start 34.925 55.245) (end 46.355 55.245) (width 0.5) (layer B.Cu) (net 9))
 (segment (start 46.355 55.245) (end 48.26 57.15) (width 0.5) (layer B.Cu) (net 9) (status 800000))
 (segment (start 48.26 57.15) (end 48.1 57.31) (width 0.5) (layer B.Cu) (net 9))
 (segment (start 48.1 57.31) (end 45.72 57.31) (width 0.5) (layer B.Cu) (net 9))
 (segment (start 33.02 57.15) (end 32.86 57.31) (width 0.5) (layer B.Cu) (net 9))
 (segment (start 32.86 57.31) (end 30.48 57.31) (width 0.5) (layer B.Cu) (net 9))
 (segment (start 17.78 57.15) (end 17.62 57.31) (width 0.5) (layer B.Cu) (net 9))
 (segment (start 17.62 57.31) (end 15.24 57.31) (width 0.5) (layer B.Cu) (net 9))
 (segment (start 3.85064 38.5699) (end 3.85064 49.73064) (width 0.5) (layer B.Cu) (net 2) (status 400000))
 (segment (start 3.85064 49.73064) (end 11.43 57.31) (width 0.5) (layer B.Cu) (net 2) (status 800000))
 (segment (start 51.435 59.69) (end 51.435 62.23) (width 0.5) (layer B.Cu) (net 2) (status C00000))
 (segment (start 38.1 57.15) (end 41.75 57.15) (width 0.5) (layer B.Cu) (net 2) (status 800000))
 (segment (start 41.75 57.15) (end 41.91 57.31) (width 0.5) (layer B.Cu) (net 2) (status C00000))
 (segment (start 26.67 57.31) (end 24.765 59.215) (width 0.5) (layer B.Cu) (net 2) (status 400000))
 (segment (start 34.925 57.15) (end 38.1 57.15) (width 0.5) (layer B.Cu) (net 2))
 (segment (start 32.385 59.69) (end 34.925 57.15) (width 0.5) (layer B.Cu) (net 2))
 (via (at 32.385 59.69) (size 1.5) (drill 0.8) (layers F.Cu B.Cu) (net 2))
 (segment (start 24.765 59.69) (end 32.385 59.69) (width 0.5) (layer F.Cu) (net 2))
 (via (at 24.765 59.69) (size 1.5) (drill 0.8) (layers F.Cu B.Cu) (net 2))
 (segment (start 24.765 59.215) (end 24.765 59.69) (width 0.5) (layer B.Cu) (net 2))
 (segment (start 38.1 64.135) (end 38.1 62.23) (width 0.5) (layer B.Cu) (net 2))
 (via (at 38.1 62.23) (size 1.5) (drill 0.8) (layers F.Cu B.Cu) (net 2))
 (segment (start 38.1 62.23) (end 38.1 57.15) (width 0.5) (layer F.Cu) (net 2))
 (via (at 38.1 57.15) (size 1.5) (drill 0.8) (layers F.Cu B.Cu) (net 2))
 (segment (start 38.1 57.15) (end 38.1 57.31) (width 0.5) (layer B.Cu) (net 2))
 (segment (start 38.1 57.31) (end 38.1 57.15) (width 0.5) (layer B.Cu) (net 2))
 (segment (start 38.1 57.15) (end 38.1 57.31) (width 0.5) (layer B.Cu) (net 2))
 (segment (start 26.67 57.31) (end 26.67 57.785) (width 0.5) (layer B.Cu) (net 2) (status C00000))
 (segment (start 11.43 57.31) (end 11.43 58.42) (width 0.5) (layer B.Cu) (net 2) (status 400000))
 (segment (start 49.53 64.135) (end 51.435 62.23) (width 0.5) (layer B.Cu) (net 2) (status 800000))
 (segment (start 17.145 64.135) (end 38.1 64.135) (width 0.5) (layer B.Cu) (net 2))
 (segment (start 38.1 64.135) (end 49.53 64.135) (width 0.5) (layer B.Cu) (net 2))
 (segment (start 11.43 58.42) (end 17.145 64.135) (width 0.5) (layer B.Cu) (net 2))
 (segment (start 12.7 57.31) (end 12.7 58.42) (width 0.5) (layer B.Cu) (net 11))
 (segment (start 20.32 60.325) (end 22.225 62.23) (width 0.5) (layer B.Cu) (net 11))
 (segment (start 14.605 60.325) (end 20.32 60.325) (width 0.5) (layer B.Cu) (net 11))
 (segment (start 12.7 58.42) (end 14.605 60.325) (width 0.5) (layer B.Cu) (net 11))
 (segment (start 13.97 57.31) (end 13.97 58.42) (width 0.5) (layer B.Cu) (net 12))
 (segment (start 21.59 59.055) (end 24.765 62.23) (width 0.5) (layer B.Cu) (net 12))
 (segment (start 14.605 59.055) (end 21.59 59.055) (width 0.5) (layer B.Cu) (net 12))
 (segment (start 13.97 58.42) (end 14.605 59.055) (width 0.5) (layer B.Cu) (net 12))
 (segment (start 27.94 57.31) (end 27.94 61.595) (width 0.5) (layer B.Cu) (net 13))
 (segment (start 27.94 61.595) (end 27.305 62.23) (width 0.5) (layer B.Cu) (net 13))
 (segment (start 29.21 57.31) (end 29.21 61.595) (width 0.5) (layer B.Cu) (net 14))
 (segment (start 29.21 61.595) (end 29.845 62.23) (width 0.5) (layer B.Cu) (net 14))
 (segment (start 43.18 57.31) (end 43.18 57.785) (width 0.5) (layer B.Cu) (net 15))
 (segment (start 43.18 57.785) (end 41.91 59.055) (width 0.5) (layer B.Cu) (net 15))
 (segment (start 41.91 59.055) (end 35.56 59.055) (width 0.5) (layer B.Cu) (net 15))
 (segment (start 35.56 59.055) (end 32.385 62.23) (width 0.5) (layer B.Cu) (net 15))
 (segment (start 44.45 57.31) (end 44.45 57.785) (width 0.5) (layer B.Cu) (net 16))
 (segment (start 44.45 57.785) (end 41.91 60.325) (width 0.5) (layer B.Cu) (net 16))
 (segment (start 41.91 60.325) (end 36.83 60.325) (width 0.5) (layer B.Cu) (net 16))
 (segment (start 36.83 60.325) (end 34.925 62.23) (width 0.5) (layer B.Cu) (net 16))
 (segment (start 44.45 39.37) (end 44.45 20.83054) (width 0.5) (layer B.Cu) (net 17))
 (segment (start 44.45 20.83054) (end 39.32936 15.7099) (width 0.5) (layer B.Cu) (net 17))
 (segment (start 44.45 46.99) (end 44.45 51.91) (width 0.5) (layer B.Cu) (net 18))
 (segment (start 36.83 39.37) (end 37.6301 38.5699) (width 0.5) (layer B.Cu) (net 19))
 (segment (start 37.6301 38.5699) (end 39.32936 38.5699) (width 0.5) (layer B.Cu) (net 19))
 (segment (start 36.83 46.99) (end 41.75 51.91) (width 0.5) (layer B.Cu) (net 20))
 (segment (start 41.75 51.91) (end 41.91 51.91) (width 0.5) (layer B.Cu) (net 20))
 (segment (start 24.08936 15.7099) (end 29.21 20.83054) (width 0.5) (layer B.Cu) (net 21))
 (segment (start 29.21 20.83054) (end 29.21 39.37) (width 0.5) (layer B.Cu) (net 21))
 (segment (start 29.21 46.99) (end 29.21 51.91) (width 0.5) (layer B.Cu) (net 22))
 (segment (start 21.59 39.37) (end 22.3901 38.5699) (width 0.5) (layer B.Cu) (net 23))
 (segment (start 22.3901 38.5699) (end 24.08936 38.5699) (width 0.5) (layer B.Cu) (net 23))
 (segment (start 21.59 46.99) (end 26.51 51.91) (width 0.5) (layer B.Cu) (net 24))
 (segment (start 26.51 51.91) (end 26.67 51.91) (width 0.5) (layer B.Cu) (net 24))
 (segment (start 13.97 39.37) (end 13.97 20.83054) (width 0.5) (layer B.Cu) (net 25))
 (segment (start 13.97 20.83054) (end 8.84936 15.7099) (width 0.5) (layer B.Cu) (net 25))
 (segment (start 13.97 46.99) (end 13.97 51.91) (width 0.5) (layer B.Cu) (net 26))
 (segment (start 6.35 39.37) (end 7.1501 38.5699) (width 0.5) (layer B.Cu) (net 1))
 (segment (start 7.1501 38.5699) (end 8.84936 38.5699) (width 0.5) (layer B.Cu) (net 1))
 (segment (start 6.35 46.99) (end 11.27 51.91) (width 0.5) (layer B.Cu) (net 27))
 (segment (start 11.27 51.91) (end 11.43 51.91) (width 0.5) (layer B.Cu) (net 27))
 (segment (start 48.26 49.53) (end 46.05 49.53) (width 0.5) (layer B.Cu) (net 4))
 (segment (start 46.05 49.53) (end 45.72 49.86) (width 0.5) (layer B.Cu) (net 4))
 (segment (start 45.72 49.86) (end 45.72 51.91) (width 0.5) (layer B.Cu) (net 4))
 (segment (start 33.02 49.53) (end 30.81 49.53) (width 0.5) (layer B.Cu) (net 6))
 (segment (start 30.81 49.53) (end 30.48 49.86) (width 0.5) (layer B.Cu) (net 6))
 (segment (start 30.48 49.86) (end 30.48 51.91) (width 0.5) (layer B.Cu) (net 6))
 (segment (start 17.78 49.53) (end 15.57 49.53) (width 0.5) (layer B.Cu) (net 8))
 (segment (start 15.57 49.53) (end 15.24 49.86) (width 0.5) (layer B.Cu) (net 8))
 (segment (start 15.24 49.86) (end 15.24 51.91) (width 0.5) (layer B.Cu) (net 8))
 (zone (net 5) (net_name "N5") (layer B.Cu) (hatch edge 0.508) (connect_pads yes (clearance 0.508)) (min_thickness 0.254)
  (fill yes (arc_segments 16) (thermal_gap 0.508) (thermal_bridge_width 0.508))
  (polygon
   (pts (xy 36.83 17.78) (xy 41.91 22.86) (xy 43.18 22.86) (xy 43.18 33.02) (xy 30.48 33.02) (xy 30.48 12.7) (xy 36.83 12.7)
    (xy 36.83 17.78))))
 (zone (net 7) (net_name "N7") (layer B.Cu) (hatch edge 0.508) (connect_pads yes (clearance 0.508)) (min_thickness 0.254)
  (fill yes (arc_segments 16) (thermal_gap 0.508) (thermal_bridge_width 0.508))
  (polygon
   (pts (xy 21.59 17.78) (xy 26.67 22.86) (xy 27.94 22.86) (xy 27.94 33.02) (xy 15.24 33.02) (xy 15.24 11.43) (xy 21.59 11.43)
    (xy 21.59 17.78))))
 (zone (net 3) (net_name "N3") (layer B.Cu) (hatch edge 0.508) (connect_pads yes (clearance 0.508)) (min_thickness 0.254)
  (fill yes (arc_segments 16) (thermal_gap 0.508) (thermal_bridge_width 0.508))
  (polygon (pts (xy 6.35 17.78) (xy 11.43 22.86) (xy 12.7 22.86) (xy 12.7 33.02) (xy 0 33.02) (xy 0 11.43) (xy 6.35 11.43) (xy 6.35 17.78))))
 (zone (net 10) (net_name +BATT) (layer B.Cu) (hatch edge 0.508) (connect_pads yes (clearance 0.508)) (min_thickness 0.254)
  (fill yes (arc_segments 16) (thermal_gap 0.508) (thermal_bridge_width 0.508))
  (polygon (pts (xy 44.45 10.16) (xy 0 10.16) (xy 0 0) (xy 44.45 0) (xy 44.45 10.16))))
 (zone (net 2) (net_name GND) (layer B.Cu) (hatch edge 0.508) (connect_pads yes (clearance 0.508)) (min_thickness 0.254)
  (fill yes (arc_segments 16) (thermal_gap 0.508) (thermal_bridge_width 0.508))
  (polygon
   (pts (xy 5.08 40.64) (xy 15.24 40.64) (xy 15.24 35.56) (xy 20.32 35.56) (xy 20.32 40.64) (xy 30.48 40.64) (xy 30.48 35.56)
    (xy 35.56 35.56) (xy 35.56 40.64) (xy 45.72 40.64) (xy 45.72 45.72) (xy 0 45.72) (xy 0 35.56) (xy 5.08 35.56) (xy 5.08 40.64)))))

